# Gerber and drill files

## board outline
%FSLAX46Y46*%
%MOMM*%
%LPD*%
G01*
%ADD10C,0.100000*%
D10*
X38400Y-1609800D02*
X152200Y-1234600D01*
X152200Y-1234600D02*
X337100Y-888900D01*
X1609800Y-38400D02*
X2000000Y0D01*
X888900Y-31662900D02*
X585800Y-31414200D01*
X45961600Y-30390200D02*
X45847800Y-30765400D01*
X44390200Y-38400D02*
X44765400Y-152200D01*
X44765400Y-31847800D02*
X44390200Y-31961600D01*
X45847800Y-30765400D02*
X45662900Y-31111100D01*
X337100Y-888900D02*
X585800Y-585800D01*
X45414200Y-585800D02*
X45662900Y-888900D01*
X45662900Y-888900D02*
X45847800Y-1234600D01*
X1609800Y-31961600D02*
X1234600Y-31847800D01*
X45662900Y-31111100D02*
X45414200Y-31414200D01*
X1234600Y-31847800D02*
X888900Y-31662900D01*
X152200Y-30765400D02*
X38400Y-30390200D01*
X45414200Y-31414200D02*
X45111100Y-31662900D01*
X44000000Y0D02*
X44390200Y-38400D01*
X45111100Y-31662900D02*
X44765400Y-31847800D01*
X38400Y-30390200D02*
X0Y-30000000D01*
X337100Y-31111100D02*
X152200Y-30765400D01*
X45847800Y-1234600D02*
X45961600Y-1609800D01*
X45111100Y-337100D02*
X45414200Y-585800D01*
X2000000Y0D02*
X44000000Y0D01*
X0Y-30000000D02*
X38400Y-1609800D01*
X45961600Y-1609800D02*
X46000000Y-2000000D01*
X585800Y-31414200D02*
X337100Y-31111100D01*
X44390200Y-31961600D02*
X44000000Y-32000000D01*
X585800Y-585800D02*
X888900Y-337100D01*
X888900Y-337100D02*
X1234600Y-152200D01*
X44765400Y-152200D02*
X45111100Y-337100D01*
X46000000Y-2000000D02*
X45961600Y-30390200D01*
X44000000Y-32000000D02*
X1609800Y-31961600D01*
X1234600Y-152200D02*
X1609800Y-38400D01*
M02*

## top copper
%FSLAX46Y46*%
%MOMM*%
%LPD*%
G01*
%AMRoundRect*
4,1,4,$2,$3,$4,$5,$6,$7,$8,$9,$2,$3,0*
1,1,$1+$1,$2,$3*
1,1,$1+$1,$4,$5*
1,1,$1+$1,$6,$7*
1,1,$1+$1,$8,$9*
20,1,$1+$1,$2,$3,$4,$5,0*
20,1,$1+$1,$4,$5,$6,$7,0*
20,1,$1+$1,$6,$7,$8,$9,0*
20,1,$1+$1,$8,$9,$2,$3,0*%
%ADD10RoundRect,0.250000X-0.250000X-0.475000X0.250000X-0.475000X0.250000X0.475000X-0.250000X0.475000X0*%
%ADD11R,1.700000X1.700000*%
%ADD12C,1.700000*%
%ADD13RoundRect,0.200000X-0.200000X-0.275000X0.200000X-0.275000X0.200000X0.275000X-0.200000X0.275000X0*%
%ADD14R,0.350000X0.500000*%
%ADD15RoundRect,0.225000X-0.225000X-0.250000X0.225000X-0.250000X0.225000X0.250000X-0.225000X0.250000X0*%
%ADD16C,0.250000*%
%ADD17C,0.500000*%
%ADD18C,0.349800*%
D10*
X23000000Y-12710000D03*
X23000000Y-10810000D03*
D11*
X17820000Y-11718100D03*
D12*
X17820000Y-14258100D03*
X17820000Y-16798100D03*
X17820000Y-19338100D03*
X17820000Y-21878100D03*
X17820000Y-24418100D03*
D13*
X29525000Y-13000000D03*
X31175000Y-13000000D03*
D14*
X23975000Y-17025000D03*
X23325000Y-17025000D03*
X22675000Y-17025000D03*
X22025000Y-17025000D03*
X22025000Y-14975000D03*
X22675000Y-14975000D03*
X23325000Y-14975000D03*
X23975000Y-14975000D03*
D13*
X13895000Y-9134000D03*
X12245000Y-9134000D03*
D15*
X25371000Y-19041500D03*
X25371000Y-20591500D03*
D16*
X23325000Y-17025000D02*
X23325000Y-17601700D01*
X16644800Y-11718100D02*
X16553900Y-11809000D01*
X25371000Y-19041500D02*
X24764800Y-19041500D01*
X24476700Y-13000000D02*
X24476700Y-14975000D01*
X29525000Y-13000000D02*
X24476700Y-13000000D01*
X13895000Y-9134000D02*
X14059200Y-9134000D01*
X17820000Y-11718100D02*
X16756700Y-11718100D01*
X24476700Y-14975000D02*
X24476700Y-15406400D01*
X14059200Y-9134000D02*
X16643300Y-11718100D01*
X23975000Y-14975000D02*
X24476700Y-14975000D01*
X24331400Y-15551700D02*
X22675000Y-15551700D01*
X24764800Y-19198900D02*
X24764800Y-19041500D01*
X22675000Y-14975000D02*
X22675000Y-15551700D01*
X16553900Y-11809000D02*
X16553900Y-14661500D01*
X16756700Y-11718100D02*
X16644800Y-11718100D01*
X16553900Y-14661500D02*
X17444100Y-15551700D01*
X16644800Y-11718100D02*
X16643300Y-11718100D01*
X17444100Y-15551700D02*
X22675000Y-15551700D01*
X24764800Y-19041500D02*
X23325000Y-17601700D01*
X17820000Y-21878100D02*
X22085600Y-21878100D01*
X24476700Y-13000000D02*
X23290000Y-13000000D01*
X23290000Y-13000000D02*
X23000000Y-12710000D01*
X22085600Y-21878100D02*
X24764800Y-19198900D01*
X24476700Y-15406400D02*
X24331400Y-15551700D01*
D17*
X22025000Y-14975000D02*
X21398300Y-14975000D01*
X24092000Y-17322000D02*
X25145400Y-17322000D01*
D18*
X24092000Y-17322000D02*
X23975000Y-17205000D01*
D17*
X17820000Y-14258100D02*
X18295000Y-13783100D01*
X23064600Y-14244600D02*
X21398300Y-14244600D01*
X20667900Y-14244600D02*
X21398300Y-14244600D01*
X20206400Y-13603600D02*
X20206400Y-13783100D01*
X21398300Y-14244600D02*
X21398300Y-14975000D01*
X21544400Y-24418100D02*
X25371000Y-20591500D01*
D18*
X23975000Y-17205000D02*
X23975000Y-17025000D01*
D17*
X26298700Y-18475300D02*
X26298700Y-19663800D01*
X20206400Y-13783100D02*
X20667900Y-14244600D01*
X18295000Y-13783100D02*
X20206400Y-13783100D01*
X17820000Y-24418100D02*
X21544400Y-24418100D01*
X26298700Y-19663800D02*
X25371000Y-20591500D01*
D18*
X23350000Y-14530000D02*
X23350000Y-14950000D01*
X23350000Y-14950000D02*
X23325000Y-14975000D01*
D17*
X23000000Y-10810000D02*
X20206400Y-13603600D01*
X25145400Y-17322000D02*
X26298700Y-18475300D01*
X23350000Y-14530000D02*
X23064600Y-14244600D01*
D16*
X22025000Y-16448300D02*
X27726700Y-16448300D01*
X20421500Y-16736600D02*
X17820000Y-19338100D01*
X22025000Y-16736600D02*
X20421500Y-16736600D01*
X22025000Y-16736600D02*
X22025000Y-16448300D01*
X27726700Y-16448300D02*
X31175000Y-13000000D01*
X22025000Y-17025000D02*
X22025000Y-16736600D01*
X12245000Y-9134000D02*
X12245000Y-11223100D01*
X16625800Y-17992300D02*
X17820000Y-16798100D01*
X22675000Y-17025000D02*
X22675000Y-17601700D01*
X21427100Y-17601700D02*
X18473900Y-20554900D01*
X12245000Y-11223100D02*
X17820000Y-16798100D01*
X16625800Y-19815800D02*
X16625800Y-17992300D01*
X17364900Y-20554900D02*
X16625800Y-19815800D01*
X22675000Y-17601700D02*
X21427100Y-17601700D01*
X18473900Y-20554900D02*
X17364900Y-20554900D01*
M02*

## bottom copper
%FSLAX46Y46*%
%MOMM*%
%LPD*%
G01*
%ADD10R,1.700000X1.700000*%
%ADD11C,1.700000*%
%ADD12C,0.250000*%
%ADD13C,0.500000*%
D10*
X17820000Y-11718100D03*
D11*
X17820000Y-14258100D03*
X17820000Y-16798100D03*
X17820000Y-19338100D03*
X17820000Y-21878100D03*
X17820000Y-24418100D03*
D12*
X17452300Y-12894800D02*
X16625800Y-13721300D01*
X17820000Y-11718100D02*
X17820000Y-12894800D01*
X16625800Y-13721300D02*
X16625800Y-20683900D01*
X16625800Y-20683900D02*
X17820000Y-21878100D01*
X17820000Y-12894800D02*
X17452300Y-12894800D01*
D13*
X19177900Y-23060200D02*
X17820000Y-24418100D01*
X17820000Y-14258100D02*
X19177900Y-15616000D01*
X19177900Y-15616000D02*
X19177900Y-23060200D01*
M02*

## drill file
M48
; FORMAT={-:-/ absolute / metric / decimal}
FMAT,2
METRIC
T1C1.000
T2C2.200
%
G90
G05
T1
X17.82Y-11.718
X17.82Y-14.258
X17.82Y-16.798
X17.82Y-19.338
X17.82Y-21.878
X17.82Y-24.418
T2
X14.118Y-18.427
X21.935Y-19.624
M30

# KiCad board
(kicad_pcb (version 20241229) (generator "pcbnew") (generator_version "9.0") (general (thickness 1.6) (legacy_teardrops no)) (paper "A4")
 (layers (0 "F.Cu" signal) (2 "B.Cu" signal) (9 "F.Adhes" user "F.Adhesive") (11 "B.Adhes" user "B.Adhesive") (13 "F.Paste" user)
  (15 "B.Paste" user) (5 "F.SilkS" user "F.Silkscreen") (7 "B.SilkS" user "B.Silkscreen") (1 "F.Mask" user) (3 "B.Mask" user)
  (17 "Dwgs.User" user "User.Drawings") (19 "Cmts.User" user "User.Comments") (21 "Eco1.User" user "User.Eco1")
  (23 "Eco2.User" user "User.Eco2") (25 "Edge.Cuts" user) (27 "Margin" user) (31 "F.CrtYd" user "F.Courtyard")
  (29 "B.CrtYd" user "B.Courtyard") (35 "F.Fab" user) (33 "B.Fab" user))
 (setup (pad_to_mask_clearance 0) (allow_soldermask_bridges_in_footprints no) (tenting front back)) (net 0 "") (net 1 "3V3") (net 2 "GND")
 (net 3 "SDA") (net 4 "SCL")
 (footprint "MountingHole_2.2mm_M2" (layer "F.Cu") (at 21.9348 19.624)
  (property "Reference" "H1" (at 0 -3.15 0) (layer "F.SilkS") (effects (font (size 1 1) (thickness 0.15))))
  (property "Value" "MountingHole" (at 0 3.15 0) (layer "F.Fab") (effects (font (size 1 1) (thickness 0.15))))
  (pad "" np_thru_hole circle (at 0 0) (size 2.2 2.2) (drill 2.2) (layers "*.Cu" "*.Mask")))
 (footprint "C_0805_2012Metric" (layer "F.Cu") (at 23 11.76 90)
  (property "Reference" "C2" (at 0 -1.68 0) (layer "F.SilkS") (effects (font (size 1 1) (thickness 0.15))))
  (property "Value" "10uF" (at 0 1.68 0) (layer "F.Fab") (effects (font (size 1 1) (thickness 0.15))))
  (pad "1" smd roundrect (at -0.95 0) (size 1 1.45) (layers "F.Cu" "F.Mask" "F.Paste") (roundrect_rratio 0.25) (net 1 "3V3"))
  (pad "2" smd roundrect (at 0.95 0) (size 1 1.45) (layers "F.Cu" "F.Mask" "F.Paste") (roundrect_rratio 0.25) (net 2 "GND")))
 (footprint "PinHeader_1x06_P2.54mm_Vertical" (layer "F.Cu") (at 17.82 11.7181)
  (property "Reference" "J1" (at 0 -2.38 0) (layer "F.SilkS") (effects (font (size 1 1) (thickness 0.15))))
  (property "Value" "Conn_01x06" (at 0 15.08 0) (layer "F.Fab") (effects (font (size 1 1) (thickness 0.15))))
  (pad "1" thru_hole rect (at 0 0) (size 1.7 1.7) (drill 1) (layers "*.Cu" "*.Mask") (remove_unused_layers no) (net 1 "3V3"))
  (pad "2" thru_hole circle (at 0 2.54) (size 1.7 1.7) (drill 1) (layers "*.Cu" "*.Mask") (remove_unused_layers no) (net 2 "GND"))
  (pad "3" thru_hole circle (at 0 5.08) (size 1.7 1.7) (drill 1) (layers "*.Cu" "*.Mask") (remove_unused_layers no) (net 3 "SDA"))
  (pad "4" thru_hole circle (at 0 7.62) (size 1.7 1.7) (drill 1) (layers "*.Cu" "*.Mask") (remove_unused_layers no) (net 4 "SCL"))
  (pad "5" thru_hole circle (at 0 10.16) (size 1.7 1.7) (drill 1) (layers "*.Cu" "*.Mask") (remove_unused_layers no) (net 1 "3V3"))
  (pad "6" thru_hole circle (at 0 12.7) (size 1.7 1.7) (drill 1) (layers "*.Cu" "*.Mask") (remove_unused_layers no) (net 2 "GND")))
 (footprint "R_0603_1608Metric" (layer "F.Cu") (at 30.35 13)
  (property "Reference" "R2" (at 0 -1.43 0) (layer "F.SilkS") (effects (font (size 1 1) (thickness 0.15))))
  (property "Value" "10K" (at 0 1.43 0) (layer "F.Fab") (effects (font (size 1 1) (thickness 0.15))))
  (pad "1" smd roundrect (at -0.825 0) (size 0.8 0.95) (layers "F.Cu" "F.Mask" "F.Paste") (roundrect_rratio 0.25) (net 1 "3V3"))
  (pad "2" smd roundrect (at 0.825 0) (size 0.8 0.95) (layers "F.Cu" "F.Mask" "F.Paste") (roundrect_rratio 0.25) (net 4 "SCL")))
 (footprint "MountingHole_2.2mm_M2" (layer "F.Cu") (at 14.1183 18.4265)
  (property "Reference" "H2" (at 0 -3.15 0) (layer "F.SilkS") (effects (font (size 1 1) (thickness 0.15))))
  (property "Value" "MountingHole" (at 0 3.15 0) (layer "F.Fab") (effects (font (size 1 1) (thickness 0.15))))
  (pad "" np_thru_hole circle (at 0 0) (size 2.2 2.2) (drill 2.2) (layers "*.Cu" "*.Mask")))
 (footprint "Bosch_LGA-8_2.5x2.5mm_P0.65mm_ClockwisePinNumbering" (layer "F.Cu") (at 23 16 180)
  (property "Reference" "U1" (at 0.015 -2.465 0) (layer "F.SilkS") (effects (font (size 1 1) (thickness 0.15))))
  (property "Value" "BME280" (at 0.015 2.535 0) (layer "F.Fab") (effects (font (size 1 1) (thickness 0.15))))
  (pad "1" smd rect (at -0.975 -1.025 90) (size 0.5 0.35) (layers "F.Cu" "F.Mask" "F.Paste") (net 2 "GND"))
  (pad "2" smd rect (at -0.325 -1.025 90) (size 0.5 0.35) (layers "F.Cu" "F.Mask" "F.Paste") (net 1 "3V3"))
  (pad "3" smd rect (at 0.325 -1.025 90) (size 0.5 0.35) (layers "F.Cu" "F.Mask" "F.Paste") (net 3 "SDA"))
  (pad "4" smd rect (at 0.975 -1.025 90) (size 0.5 0.35) (layers "F.Cu" "F.Mask" "F.Paste") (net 4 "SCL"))
  (pad "5" smd rect (at 0.975 1.025 90) (size 0.5 0.35) (layers "F.Cu" "F.Mask" "F.Paste") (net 2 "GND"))
  (pad "6" smd rect (at 0.325 1.025 90) (size 0.5 0.35) (layers "F.Cu" "F.Mask" "F.Paste") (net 1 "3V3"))
  (pad "7" smd rect (at -0.325 1.025 90) (size 0.5 0.35) (layers "F.Cu" "F.Mask" "F.Paste") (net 2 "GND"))
  (pad "8" smd rect (at -0.975 1.025 90) (size 0.5 0.35) (layers "F.Cu" "F.Mask" "F.Paste") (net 1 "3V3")))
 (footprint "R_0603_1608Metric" (layer "F.Cu") (at 13.07 9.134 180)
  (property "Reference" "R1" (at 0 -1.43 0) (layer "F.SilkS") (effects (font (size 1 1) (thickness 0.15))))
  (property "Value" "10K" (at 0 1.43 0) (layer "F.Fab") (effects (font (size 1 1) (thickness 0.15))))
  (pad "1" smd roundrect (at -0.825 0) (size 0.8 0.95) (layers "F.Cu" "F.Mask" "F.Paste") (roundrect_rratio 0.25) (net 1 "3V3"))
  (pad "2" smd roundrect (at 0.825 0) (size 0.8 0.95) (layers "F.Cu" "F.Mask" "F.Paste") (roundrect_rratio 0.25) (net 3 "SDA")))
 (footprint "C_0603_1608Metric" (layer "F.Cu") (at 25.371 19.8165 -90)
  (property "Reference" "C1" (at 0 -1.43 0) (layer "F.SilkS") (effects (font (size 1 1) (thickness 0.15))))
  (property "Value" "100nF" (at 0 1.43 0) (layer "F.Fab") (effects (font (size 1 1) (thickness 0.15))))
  (pad "1" smd roundrect (at -0.775 0) (size 0.9 0.95) (layers "F.Cu" "F.Mask" "F.Paste") (roundrect_rratio 0.25) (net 1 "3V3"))
  (pad "2" smd roundrect (at 0.775 0) (size 0.9 0.95) (layers "F.Cu" "F.Mask" "F.Paste") (roundrect_rratio 0.25) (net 2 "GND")))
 (gr_line (start 0.0384 1.6098) (end 0.1522 1.2346) (stroke (width 0.1) (type solid)) (layer "Edge.Cuts"))
 (gr_line (start 0.1522 1.2346) (end 0.3371 0.8889) (stroke (width 0.1) (type solid)) (layer "Edge.Cuts"))
 (gr_line (start 1.6098 0.0384) (end 2 0) (stroke (width 0.1) (type solid)) (layer "Edge.Cuts"))
 (gr_line (start 0.8889 31.6629) (end 0.5858 31.4142) (stroke (width 0.1) (type solid)) (layer "Edge.Cuts"))
 (gr_line (start 45.9616 30.3902) (end 45.8478 30.7654) (stroke (width 0.1) (type solid)) (layer "Edge.Cuts"))
 (gr_line (start 44.3902 0.0384) (end 44.7654 0.1522) (stroke (width 0.1) (type solid)) (layer "Edge.Cuts"))
 (gr_line (start 44.7654 31.8478) (end 44.3902 31.9616) (stroke (width 0.1) (type solid)) (layer "Edge.Cuts"))
 (gr_line (start 45.8478 30.7654) (end 45.6629 31.1111) (stroke (width 0.1) (type solid)) (layer "Edge.Cuts"))
 (gr_line (start 0.3371 0.8889) (end 0.5858 0.5858) (stroke (width 0.1) (type solid)) (layer "Edge.Cuts"))
 (gr_line (start 45.4142 0.5858) (end 45.6629 0.8889) (stroke (width 0.1) (type solid)) (layer "Edge.Cuts"))
 (gr_line (start 45.6629 0.8889) (end 45.8478 1.2346) (stroke (width 0.1) (type solid)) (layer "Edge.Cuts"))
 (gr_line (start 1.6098 31.9616) (end 1.2346 31.8478) (stroke (width 0.1) (type solid)) (layer "Edge.Cuts"))
 (gr_line (start 45.6629 31.1111) (end 45.4142 31.4142) (stroke (width 0.1) (type solid)) (layer "Edge.Cuts"))
 (gr_line (start 1.2346 31.8478) (end 0.8889 31.6629) (stroke (width 0.1) (type solid)) (layer "Edge.Cuts"))
 (gr_line (start 0.1522 30.7654) (end 0.0384 30.3902) (stroke (width 0.1) (type solid)) (layer "Edge.Cuts"))
 (gr_line (start 45.4142 31.4142) (end 45.1111 31.6629) (stroke (width 0.1) (type solid)) (layer "Edge.Cuts"))
 (gr_line (start 44 0) (end 44.3902 0.0384) (stroke (width 0.1) (type solid)) (layer "Edge.Cuts"))
 (gr_line (start 45.1111 31.6629) (end 44.7654 31.8478) (stroke (width 0.1) (type solid)) (layer "Edge.Cuts"))
 (gr_line (start 0.0384 30.3902) (end 0 30) (stroke (width 0.1) (type solid)) (layer "Edge.Cuts"))
 (gr_line (start 0.3371 31.1111) (end 0.1522 30.7654) (stroke (width 0.1) (type solid)) (layer "Edge.Cuts"))
 (gr_line (start 45.8478 1.2346) (end 45.9616 1.6098) (stroke (width 0.1) (type solid)) (layer "Edge.Cuts"))
 (gr_line (start 45.1111 0.3371) (end 45.4142 0.5858) (stroke (width 0.1) (type solid)) (layer "Edge.Cuts"))
 (gr_line (start 2 0) (end 44 0) (stroke (width 0.1) (type solid)) (layer "Edge.Cuts"))
 (gr_line (start 0 30) (end 0.0384 1.6098) (stroke (width 0.1) (type solid)) (layer "Edge.Cuts"))
 (gr_line (start 45.9616 1.6098) (end 46 2) (stroke (width 0.1) (type solid)) (layer "Edge.Cuts"))
 (gr_line (start 0.5858 31.4142) (end 0.3371 31.1111) (stroke (width 0.1) (type solid)) (layer "Edge.Cuts"))
 (gr_line (start 44.3902 31.9616) (end 44 32) (stroke (width 0.1) (type solid)) (layer "Edge.Cuts"))
 (gr_line (start 0.5858 0.5858) (end 0.8889 0.3371) (stroke (width 0.1) (type solid)) (layer "Edge.Cuts"))
 (gr_line (start 0.8889 0.3371) (end 1.2346 0.1522) (stroke (width 0.1) (type solid)) (layer "Edge.Cuts"))
 (gr_line (start 44.7654 0.1522) (end 45.1111 0.3371) (stroke (width 0.1) (type solid)) (layer "Edge.Cuts"))
 (gr_line (start 46 2) (end 45.9616 30.3902) (stroke (width 0.1) (type solid)) (layer "Edge.Cuts"))
 (gr_line (start 44 32) (end 1.6098 31.9616) (stroke (width 0.1) (type solid)) (layer "Edge.Cuts"))
 (gr_line (start 1.2346 0.1522) (end 1.6098 0.0384) (stroke (width 0.1) (type solid)) (layer "Edge.Cuts"))
 (segment (start 23.325 17.025) (end 23.325 17.6017) (width 0.25) (layer "F.Cu") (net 1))
 (segment (start 16.6448 11.7181) (end 16.5539 11.809) (width 0.25) (layer "F.Cu") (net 1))
 (segment (start 25.371 19.0415) (end 24.7648 19.0415) (width 0.25) (layer "F.Cu") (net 1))
 (segment (start 24.4767 13) (end 24.4767 14.975) (width 0.25) (layer "F.Cu") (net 1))
 (segment (start 29.525 13) (end 24.4767 13) (width 0.25) (layer "F.Cu") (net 1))
 (segment (start 13.895 9.134) (end 14.0592 9.134) (width 0.25) (layer "F.Cu") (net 1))
 (segment (start 17.82 11.7181) (end 16.7567 11.7181) (width 0.25) (layer "F.Cu") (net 1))
 (segment (start 24.4767 14.975) (end 24.4767 15.4064) (width 0.25) (layer "F.Cu") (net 1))
 (segment (start 14.0592 9.134) (end 16.6433 11.7181) (width 0.25) (layer "F.Cu") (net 1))
 (segment (start 23.975 14.975) (end 24.4767 14.975) (width 0.25) (layer "F.Cu") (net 1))
 (segment (start 24.3314 15.5517) (end 22.675 15.5517) (width 0.25) (layer "F.Cu") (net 1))
 (segment (start 24.7648 19.1989) (end 24.7648 19.0415) (width 0.25) (layer "F.Cu") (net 1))
 (segment (start 22.675 14.975) (end 22.675 15.5517) (width 0.25) (layer "F.Cu") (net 1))
 (segment (start 16.5539 11.809) (end 16.5539 14.6615) (width 0.25) (layer "F.Cu") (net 1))
 (segment (start 16.7567 11.7181) (end 16.6448 11.7181) (width 0.25) (layer "F.Cu") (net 1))
 (segment (start 16.5539 14.6615) (end 17.4441 15.5517) (width 0.25) (layer "F.Cu") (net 1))
 (segment (start 16.6448 11.7181) (end 16.6433 11.7181) (width 0.25) (layer "F.Cu") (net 1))
 (segment (start 17.4441 15.5517) (end 22.675 15.5517) (width 0.25) (layer "F.Cu") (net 1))
 (segment (start 24.7648 19.0415) (end 23.325 17.6017) (width 0.25) (layer "F.Cu") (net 1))
 (segment (start 17.82 21.8781) (end 22.0856 21.8781) (width 0.25) (layer "F.Cu") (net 1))
 (segment (start 24.4767 13) (end 23.29 13) (width 0.25) (layer "F.Cu") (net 1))
 (segment (start 23.29 13) (end 23 12.71) (width 0.25) (layer "F.Cu") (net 1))
 (segment (start 22.0856 21.8781) (end 24.7648 19.1989) (width 0.25) (layer "F.Cu") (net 1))
 (segment (start 24.4767 15.4064) (end 24.3314 15.5517) (width 0.25) (layer "F.Cu") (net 1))
 (segment (start 17.4523 12.8948) (end 16.6258 13.7213) (width 0.25) (layer "B.Cu") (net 1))
 (segment (start 17.82 11.7181) (end 17.82 12.8948) (width 0.25) (layer "B.Cu") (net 1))
 (segment (start 16.6258 13.7213) (end 16.6258 20.6839) (width 0.25) (layer "B.Cu") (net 1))
 (segment (start 16.6258 20.6839) (end 17.82 21.8781) (width 0.25) (layer "B.Cu") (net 1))
 (segment (start 17.82 12.8948) (end 17.4523 12.8948) (width 0.25) (layer "B.Cu") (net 1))
 (segment (start 22.025 14.975) (end 21.3983 14.975) (width 0.5) (layer "F.Cu") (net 2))
 (segment (start 24.092 17.322) (end 25.1454 17.322) (width 0.5) (layer "F.Cu") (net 2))
 (segment (start 24.092 17.322) (end 23.975 17.205) (width 0.3498) (layer "F.Cu") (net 2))
 (segment (start 17.82 14.2581) (end 18.295 13.7831) (width 0.5) (layer "F.Cu") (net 2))
 (segment (start 23.0646 14.2446) (end 21.3983 14.2446) (width 0.5) (layer "F.Cu") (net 2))
 (segment (start 20.6679 14.2446) (end 21.3983 14.2446) (width 0.5) (layer "F.Cu") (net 2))
 (segment (start 20.2064 13.6036) (end 20.2064 13.7831) (width 0.5) (layer "F.Cu") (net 2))
 (segment (start 21.3983 14.2446) (end 21.3983 14.975) (width 0.5) (layer "F.Cu") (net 2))
 (segment (start 21.5444 24.4181) (end 25.371 20.5915) (width 0.5) (layer "F.Cu") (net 2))
 (segment (start 23.975 17.205) (end 23.975 17.025) (width 0.3498) (layer "F.Cu") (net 2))
 (segment (start 26.2987 18.4753) (end 26.2987 19.6638) (width 0.5) (layer "F.Cu") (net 2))
 (segment (start 20.2064 13.7831) (end 20.6679 14.2446) (width 0.5) (layer "F.Cu") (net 2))
 (segment (start 18.295 13.7831) (end 20.2064 13.7831) (width 0.5) (layer "F.Cu") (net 2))
 (segment (start 17.82 24.4181) (end 21.5444 24.4181) (width 0.5) (layer "F.Cu") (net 2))
 (segment (start 26.2987 19.6638) (end 25.371 20.5915) (width 0.5) (layer "F.Cu") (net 2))
 (segment (start 23.35 14.53) (end 23.35 14.95) (width 0.3498) (layer "F.Cu") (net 2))
 (segment (start 23.35 14.95) (end 23.325 14.975) (width 0.3498) (layer "F.Cu") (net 2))
 (segment (start 23 10.81) (end 20.2064 13.6036) (width 0.5) (layer "F.Cu") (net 2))
 (segment (start 25.1454 17.322) (end 26.2987 18.4753) (width 0.5) (layer "F.Cu") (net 2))
 (segment (start 23.35 14.53) (end 23.0646 14.2446) (width 0.5) (layer "F.Cu") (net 2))
 (segment (start 19.1779 23.0602) (end 17.82 24.4181) (width 0.5) (layer "B.Cu") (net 2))
 (segment (start 17.82 14.2581) (end 19.1779 15.616) (width 0.5) (layer "B.Cu") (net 2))
 (segment (start 19.1779 15.616) (end 19.1779 23.0602) (width 0.5) (layer "B.Cu") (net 2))
 (segment (start 22.025 16.4483) (end 27.7267 16.4483) (width 0.25) (layer "F.Cu") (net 4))
 (segment (start 20.4215 16.7366) (end 17.82 19.3381) (width 0.25) (layer "F.Cu") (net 4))
 (segment (start 22.025 16.7366) (end 20.4215 16.7366) (width 0.25) (layer "F.Cu") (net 4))
 (segment (start 22.025 16.7366) (end 22.025 16.4483) (width 0.25) (layer "F.Cu") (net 4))
 (segment (start 27.7267 16.4483) (end 31.175 13) (width 0.25) (layer "F.Cu") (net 4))
 (segment (start 22.025 17.025) (end 22.025 16.7366) (width 0.25) (layer "F.Cu") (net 4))
 (segment (start 12.245 9.134) (end 12.245 11.2231) (width 0.25) (layer "F.Cu") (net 3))
 (segment (start 16.6258 17.9923) (end 17.82 16.7981) (width 0.25) (layer "F.Cu") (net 3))
 (segment (start 22.675 17.025) (end 22.675 17.6017) (width 0.25) (layer "F.Cu") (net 3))
 (segment (start 21.4271 17.6017) (end 18.4739 20.5549) (width 0.25) (layer "F.Cu") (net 3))
 (segment (start 12.245 11.2231) (end 17.82 16.7981) (width 0.25) (layer "F.Cu") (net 3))
 (segment (start 16.6258 19.8158) (end 16.6258 17.9923) (width 0.25) (layer "F.Cu") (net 3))
 (segment (start 17.3649 20.5549) (end 16.6258 19.8158) (width 0.25) (layer "F.Cu") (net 3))
 (segment (start 22.675 17.6017) (end 21.4271 17.6017) (width 0.25) (layer "F.Cu") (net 3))
 (segment (start 18.4739 20.5549) (end 17.3649 20.5549) (width 0.25) (layer "F.Cu") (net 3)))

